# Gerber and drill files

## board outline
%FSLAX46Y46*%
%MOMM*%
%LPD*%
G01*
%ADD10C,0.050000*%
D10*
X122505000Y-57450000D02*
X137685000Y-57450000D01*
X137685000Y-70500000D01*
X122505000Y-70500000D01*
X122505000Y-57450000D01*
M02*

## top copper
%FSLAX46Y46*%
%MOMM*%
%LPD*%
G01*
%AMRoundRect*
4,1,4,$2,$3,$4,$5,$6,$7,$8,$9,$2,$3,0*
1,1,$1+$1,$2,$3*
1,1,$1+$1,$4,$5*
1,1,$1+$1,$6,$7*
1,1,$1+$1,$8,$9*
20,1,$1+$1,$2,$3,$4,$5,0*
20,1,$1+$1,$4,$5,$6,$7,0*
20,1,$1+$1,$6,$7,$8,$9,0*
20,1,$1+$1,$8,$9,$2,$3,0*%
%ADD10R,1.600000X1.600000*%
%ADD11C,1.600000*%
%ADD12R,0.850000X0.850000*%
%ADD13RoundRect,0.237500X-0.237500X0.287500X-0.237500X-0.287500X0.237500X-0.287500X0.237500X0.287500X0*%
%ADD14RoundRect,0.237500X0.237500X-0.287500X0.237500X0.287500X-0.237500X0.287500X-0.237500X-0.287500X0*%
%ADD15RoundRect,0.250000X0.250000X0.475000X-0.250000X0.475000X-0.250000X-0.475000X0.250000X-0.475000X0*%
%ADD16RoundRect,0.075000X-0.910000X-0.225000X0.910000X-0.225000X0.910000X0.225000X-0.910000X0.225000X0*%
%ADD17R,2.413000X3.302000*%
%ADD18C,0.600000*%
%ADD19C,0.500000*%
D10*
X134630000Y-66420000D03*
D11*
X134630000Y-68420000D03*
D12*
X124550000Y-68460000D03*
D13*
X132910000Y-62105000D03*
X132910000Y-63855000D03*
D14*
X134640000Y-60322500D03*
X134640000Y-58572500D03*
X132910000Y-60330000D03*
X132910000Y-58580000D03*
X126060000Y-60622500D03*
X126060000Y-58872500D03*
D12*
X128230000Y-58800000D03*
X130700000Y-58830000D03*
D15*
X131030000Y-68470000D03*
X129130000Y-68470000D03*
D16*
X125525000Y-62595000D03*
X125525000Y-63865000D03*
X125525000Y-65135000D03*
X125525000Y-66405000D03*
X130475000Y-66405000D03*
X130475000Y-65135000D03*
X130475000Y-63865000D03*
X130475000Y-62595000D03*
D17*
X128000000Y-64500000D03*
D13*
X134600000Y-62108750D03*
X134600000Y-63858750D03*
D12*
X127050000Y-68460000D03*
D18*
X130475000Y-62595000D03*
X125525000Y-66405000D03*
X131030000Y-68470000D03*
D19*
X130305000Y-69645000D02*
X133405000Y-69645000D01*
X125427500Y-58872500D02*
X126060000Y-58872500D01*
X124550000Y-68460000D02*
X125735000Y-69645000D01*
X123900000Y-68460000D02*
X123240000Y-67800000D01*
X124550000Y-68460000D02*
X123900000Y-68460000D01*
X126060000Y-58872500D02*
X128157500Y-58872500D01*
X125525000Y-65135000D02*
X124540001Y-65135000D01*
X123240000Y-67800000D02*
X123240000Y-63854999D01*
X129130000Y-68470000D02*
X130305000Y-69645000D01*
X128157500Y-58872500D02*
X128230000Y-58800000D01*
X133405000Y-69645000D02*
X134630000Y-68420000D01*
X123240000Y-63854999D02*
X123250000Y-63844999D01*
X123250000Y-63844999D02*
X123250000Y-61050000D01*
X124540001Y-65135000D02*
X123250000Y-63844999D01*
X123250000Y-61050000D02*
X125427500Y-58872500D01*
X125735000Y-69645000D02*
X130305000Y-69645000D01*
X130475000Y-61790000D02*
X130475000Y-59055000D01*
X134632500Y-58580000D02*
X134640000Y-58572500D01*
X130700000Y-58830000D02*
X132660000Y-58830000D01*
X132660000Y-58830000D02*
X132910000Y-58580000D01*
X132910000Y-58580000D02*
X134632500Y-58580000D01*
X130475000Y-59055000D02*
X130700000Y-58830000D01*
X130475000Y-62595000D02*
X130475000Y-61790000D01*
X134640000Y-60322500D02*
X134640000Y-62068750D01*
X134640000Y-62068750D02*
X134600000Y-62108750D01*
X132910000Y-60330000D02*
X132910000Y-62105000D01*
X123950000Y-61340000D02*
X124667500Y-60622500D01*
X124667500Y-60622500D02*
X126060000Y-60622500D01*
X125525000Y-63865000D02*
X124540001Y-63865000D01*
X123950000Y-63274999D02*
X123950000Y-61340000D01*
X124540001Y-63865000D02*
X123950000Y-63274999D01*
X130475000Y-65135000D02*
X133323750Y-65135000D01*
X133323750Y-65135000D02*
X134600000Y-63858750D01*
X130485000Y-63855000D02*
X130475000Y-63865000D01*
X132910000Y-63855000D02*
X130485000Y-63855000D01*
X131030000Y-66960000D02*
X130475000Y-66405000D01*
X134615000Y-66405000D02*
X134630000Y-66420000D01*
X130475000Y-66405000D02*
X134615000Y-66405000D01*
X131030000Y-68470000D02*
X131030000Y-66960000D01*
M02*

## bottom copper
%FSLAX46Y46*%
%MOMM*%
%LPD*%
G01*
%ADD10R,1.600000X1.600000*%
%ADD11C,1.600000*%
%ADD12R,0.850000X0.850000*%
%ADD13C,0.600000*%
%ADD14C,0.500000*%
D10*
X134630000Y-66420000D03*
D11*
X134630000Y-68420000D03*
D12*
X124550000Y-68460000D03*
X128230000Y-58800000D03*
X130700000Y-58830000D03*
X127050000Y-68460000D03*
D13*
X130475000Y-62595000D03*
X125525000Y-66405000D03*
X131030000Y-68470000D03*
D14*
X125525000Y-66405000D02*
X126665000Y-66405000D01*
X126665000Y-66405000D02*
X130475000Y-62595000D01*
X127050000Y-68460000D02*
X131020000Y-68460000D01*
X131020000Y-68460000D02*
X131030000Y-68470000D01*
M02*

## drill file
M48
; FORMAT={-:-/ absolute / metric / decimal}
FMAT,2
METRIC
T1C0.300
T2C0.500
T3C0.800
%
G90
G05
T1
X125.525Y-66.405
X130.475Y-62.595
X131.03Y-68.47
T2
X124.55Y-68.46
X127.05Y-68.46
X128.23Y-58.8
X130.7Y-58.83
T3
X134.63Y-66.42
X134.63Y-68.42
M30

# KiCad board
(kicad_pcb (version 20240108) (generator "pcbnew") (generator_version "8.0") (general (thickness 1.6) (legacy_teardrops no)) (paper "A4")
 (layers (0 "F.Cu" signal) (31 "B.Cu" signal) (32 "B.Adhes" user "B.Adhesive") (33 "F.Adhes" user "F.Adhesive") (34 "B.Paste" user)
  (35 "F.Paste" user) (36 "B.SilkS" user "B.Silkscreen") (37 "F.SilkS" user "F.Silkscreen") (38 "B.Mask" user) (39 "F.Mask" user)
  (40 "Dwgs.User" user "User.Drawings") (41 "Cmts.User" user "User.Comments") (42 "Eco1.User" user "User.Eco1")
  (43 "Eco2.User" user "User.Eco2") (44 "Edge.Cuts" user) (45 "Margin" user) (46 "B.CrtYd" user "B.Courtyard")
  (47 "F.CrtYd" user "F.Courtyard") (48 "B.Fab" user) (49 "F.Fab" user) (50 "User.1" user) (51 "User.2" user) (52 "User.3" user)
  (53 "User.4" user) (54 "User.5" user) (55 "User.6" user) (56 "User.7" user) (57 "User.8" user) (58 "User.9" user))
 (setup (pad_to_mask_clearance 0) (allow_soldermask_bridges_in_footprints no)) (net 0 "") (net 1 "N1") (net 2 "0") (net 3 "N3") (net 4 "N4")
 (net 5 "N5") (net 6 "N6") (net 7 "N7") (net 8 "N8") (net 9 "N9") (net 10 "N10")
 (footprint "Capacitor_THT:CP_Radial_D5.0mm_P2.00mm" (layer "F.Cu") (at 134.63 66.42 -90)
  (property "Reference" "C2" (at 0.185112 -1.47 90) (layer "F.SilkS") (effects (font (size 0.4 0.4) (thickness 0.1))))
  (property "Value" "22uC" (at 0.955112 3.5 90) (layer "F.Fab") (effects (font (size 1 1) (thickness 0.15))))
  (pad "1" thru_hole rect (at 0 0 270) (size 1.6 1.6) (drill 0.8) (layers "*.Cu" "*.Mask") (remove_unused_layers no) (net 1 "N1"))
  (pad "2" thru_hole circle (at 2 0 270) (size 1.6 1.6) (drill 0.8) (layers "*.Cu" "*.Mask") (remove_unused_layers no) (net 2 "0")))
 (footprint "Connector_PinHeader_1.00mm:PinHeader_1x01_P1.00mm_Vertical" (layer "F.Cu") (at 124.55 68.46)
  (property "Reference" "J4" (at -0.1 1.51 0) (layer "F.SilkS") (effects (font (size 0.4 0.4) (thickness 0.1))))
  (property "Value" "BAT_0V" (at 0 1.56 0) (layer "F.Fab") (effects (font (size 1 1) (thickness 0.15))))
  (pad "1" thru_hole rect (at 0 0) (size 0.85 0.85) (drill 0.5) (layers "*.Cu" "*.Mask") (remove_unused_layers no) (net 2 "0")))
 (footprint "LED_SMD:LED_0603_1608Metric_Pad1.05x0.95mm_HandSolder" (layer "F.Cu") (at 132.91 62.98 -90)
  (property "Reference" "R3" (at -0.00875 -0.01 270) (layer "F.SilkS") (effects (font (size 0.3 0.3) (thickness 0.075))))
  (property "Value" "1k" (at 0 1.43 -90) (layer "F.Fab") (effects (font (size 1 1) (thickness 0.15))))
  (pad "1" smd roundrect (at -0.875 0 270) (size 1.05 0.95) (layers "F.Cu" "F.Paste" "F.Mask") (roundrect_rratio 0.25) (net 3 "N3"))
  (pad "2" smd roundrect (at 0.875 0 270) (size 1.05 0.95) (layers "F.Cu" "F.Paste" "F.Mask") (roundrect_rratio 0.25) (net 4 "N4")))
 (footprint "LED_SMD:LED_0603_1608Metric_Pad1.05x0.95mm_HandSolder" (layer "F.Cu") (at 134.64 59.4475 90)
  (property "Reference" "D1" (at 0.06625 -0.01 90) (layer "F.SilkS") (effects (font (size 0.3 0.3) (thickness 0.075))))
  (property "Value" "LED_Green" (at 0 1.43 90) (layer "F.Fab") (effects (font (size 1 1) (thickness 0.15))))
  (pad "1" smd roundrect (at -0.875 0 90) (size 1.05 0.95) (layers "F.Cu" "F.Paste" "F.Mask") (roundrect_rratio 0.25) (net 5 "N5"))
  (pad "2" smd roundrect (at 0.875 0 90) (size 1.05 0.95) (layers "F.Cu" "F.Paste" "F.Mask") (roundrect_rratio 0.25) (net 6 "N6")))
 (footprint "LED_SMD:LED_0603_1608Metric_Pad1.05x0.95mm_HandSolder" (layer "F.Cu") (at 132.91 59.455 90)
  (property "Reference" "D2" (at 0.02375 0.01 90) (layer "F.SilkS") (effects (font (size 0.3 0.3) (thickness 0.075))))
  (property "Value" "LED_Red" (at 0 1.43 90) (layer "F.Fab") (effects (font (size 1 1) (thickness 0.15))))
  (pad "1" smd roundrect (at -0.875 0 90) (size 1.05 0.95) (layers "F.Cu" "F.Paste" "F.Mask") (roundrect_rratio 0.25) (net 3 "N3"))
  (pad "2" smd roundrect (at 0.875 0 90) (size 1.05 0.95) (layers "F.Cu" "F.Paste" "F.Mask") (roundrect_rratio 0.25) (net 6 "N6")))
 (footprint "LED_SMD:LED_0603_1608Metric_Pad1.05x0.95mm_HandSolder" (layer "F.Cu") (at 126.06 59.7475 90)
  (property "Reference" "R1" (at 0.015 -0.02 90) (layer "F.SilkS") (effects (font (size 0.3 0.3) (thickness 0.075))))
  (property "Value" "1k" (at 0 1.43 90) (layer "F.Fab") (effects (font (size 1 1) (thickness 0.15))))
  (pad "1" smd roundrect (at -0.875 0 90) (size 1.05 0.95) (layers "F.Cu" "F.Paste" "F.Mask") (roundrect_rratio 0.25) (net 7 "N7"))
  (pad "2" smd roundrect (at 0.875 0 90) (size 1.05 0.95) (layers "F.Cu" "F.Paste" "F.Mask") (roundrect_rratio 0.25) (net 2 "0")))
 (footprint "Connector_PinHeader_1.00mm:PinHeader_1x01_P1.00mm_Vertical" (layer "F.Cu") (at 128.23 58.8)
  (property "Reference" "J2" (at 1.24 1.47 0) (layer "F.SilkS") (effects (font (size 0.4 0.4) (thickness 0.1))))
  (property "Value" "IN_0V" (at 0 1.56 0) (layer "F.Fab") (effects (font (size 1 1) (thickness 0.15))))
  (pad "1" thru_hole rect (at 0 0) (size 0.85 0.85) (drill 0.5) (layers "*.Cu" "*.Mask") (remove_unused_layers no) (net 2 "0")))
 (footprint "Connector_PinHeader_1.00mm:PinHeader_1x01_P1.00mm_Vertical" (layer "F.Cu") (at 130.7 58.83)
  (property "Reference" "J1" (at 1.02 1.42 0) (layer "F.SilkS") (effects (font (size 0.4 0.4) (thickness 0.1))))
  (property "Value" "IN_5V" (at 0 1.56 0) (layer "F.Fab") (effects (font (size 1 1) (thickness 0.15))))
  (pad "1" thru_hole rect (at 0 0) (size 0.85 0.85) (drill 0.5) (layers "*.Cu" "*.Mask") (remove_unused_layers no) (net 6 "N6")))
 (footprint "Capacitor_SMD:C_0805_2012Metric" (layer "F.Cu") (at 130.08 68.47 180)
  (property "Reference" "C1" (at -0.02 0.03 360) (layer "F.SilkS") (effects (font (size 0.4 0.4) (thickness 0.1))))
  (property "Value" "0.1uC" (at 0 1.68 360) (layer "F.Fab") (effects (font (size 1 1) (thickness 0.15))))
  (pad "1" smd roundrect (at -0.95 0 180) (size 1 1.45) (layers "F.Cu" "F.Paste" "F.Mask") (roundrect_rratio 0.25) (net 1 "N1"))
  (pad "2" smd roundrect (at 0.95 0 180) (size 1 1.45) (layers "F.Cu" "F.Paste" "F.Mask") (roundrect_rratio 0.25) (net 2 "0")))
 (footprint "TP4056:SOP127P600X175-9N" (layer "F.Cu") (at 128 64.5)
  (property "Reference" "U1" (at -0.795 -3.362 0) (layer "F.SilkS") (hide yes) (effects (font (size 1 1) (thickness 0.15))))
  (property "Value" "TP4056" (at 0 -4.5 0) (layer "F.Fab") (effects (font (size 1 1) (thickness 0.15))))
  (pad "1" smd roundrect (at -2.475 -1.905) (size 1.97 0.6) (layers "F.Cu" "F.Paste" "F.Mask") (roundrect_rratio 0.125) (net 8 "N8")
   (solder_mask_margin 0.102))
  (pad "2" smd roundrect (at -2.475 -0.635) (size 1.97 0.6) (layers "F.Cu" "F.Paste" "F.Mask") (roundrect_rratio 0.125) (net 7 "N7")
   (solder_mask_margin 0.102))
  (pad "3" smd roundrect (at -2.475 0.635) (size 1.97 0.6) (layers "F.Cu" "F.Paste" "F.Mask") (roundrect_rratio 0.125) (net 2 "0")
   (solder_mask_margin 0.102))
  (pad "4" smd roundrect (at -2.475 1.905) (size 1.97 0.6) (layers "F.Cu" "F.Paste" "F.Mask") (roundrect_rratio 0.125) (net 6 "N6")
   (solder_mask_margin 0.102))
  (pad "5" smd roundrect (at 2.475 1.905) (size 1.97 0.6) (layers "F.Cu" "F.Paste" "F.Mask") (roundrect_rratio 0.125) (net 1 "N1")
   (solder_mask_margin 0.102))
  (pad "6" smd roundrect (at 2.475 0.635) (size 1.97 0.6) (layers "F.Cu" "F.Paste" "F.Mask") (roundrect_rratio 0.125) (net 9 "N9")
   (solder_mask_margin 0.102))
  (pad "7" smd roundrect (at 2.475 -0.635) (size 1.97 0.6) (layers "F.Cu" "F.Paste" "F.Mask") (roundrect_rratio 0.125) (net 4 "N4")
   (solder_mask_margin 0.102))
  (pad "8" smd roundrect (at 2.475 -1.905) (size 1.97 0.6) (layers "F.Cu" "F.Paste" "F.Mask") (roundrect_rratio 0.125) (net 6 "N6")
   (solder_mask_margin 0.102))
  (pad "9" smd rect (at 0 0) (size 2.413 3.302) (layers "F.Cu" "F.Mask") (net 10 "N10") (solder_mask_margin 0.102)))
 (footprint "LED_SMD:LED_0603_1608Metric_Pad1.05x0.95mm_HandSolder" (layer "F.Cu") (at 134.6 62.98375 -90)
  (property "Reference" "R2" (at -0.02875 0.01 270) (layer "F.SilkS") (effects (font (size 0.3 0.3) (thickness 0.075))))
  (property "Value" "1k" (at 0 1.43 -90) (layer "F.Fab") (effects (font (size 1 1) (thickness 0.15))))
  (pad "1" smd roundrect (at -0.875 0 270) (size 1.05 0.95) (layers "F.Cu" "F.Paste" "F.Mask") (roundrect_rratio 0.25) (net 5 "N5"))
  (pad "2" smd roundrect (at 0.875 0 270) (size 1.05 0.95) (layers "F.Cu" "F.Paste" "F.Mask") (roundrect_rratio 0.25) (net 9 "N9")))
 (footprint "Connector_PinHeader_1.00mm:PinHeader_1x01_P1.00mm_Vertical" (layer "F.Cu") (at 127.05 68.46)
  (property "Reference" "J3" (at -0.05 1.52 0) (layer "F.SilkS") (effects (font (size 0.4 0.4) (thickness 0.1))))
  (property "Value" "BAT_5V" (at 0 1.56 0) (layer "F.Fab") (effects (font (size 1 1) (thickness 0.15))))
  (pad "1" thru_hole rect (at 0 0) (size 0.85 0.85) (drill 0.5) (layers "*.Cu" "*.Mask") (remove_unused_layers no) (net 1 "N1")))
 (gr_rect (start 122.505 57.45) (end 137.685 70.5) (stroke (width 0.05) (type default)) (fill none) (layer "Edge.Cuts"))
 (segment (start 130.305 69.645) (end 133.405 69.645) (width 0.5) (layer "F.Cu") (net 2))
 (segment (start 125.4275 58.8725) (end 126.06 58.8725) (width 0.5) (layer "F.Cu") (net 2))
 (segment (start 124.55 68.46) (end 125.735 69.645) (width 0.5) (layer "F.Cu") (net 2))
 (segment (start 123.9 68.46) (end 123.24 67.8) (width 0.5) (layer "F.Cu") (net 2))
 (segment (start 124.55 68.46) (end 123.9 68.46) (width 0.5) (layer "F.Cu") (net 2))
 (segment (start 126.06 58.8725) (end 128.1575 58.8725) (width 0.5) (layer "F.Cu") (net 2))
 (segment (start 125.525 65.135) (end 124.540001 65.135) (width 0.5) (layer "F.Cu") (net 2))
 (segment (start 123.24 67.8) (end 123.24 63.854999) (width 0.5) (layer "F.Cu") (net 2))
 (segment (start 129.13 68.47) (end 130.305 69.645) (width 0.5) (layer "F.Cu") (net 2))
 (segment (start 128.1575 58.8725) (end 128.23 58.8) (width 0.5) (layer "F.Cu") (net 2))
 (segment (start 133.405 69.645) (end 134.63 68.42) (width 0.5) (layer "F.Cu") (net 2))
 (segment (start 123.24 63.854999) (end 123.25 63.844999) (width 0.5) (layer "F.Cu") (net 2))
 (segment (start 123.25 63.844999) (end 123.25 61.05) (width 0.5) (layer "F.Cu") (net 2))
 (segment (start 124.540001 65.135) (end 123.25 63.844999) (width 0.5) (layer "F.Cu") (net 2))
 (segment (start 123.25 61.05) (end 125.4275 58.8725) (width 0.5) (layer "F.Cu") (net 2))
 (segment (start 125.735 69.645) (end 130.305 69.645) (width 0.5) (layer "F.Cu") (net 2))
 (segment (start 130.475 61.79) (end 130.475 59.055) (width 0.5) (layer "F.Cu") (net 6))
 (segment (start 134.6325 58.58) (end 134.64 58.5725) (width 0.5) (layer "F.Cu") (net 6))
 (segment (start 130.7 58.83) (end 132.66 58.83) (width 0.5) (layer "F.Cu") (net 6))
 (segment (start 132.66 58.83) (end 132.91 58.58) (width 0.5) (layer "F.Cu") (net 6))
 (segment (start 132.91 58.58) (end 134.6325 58.58) (width 0.5) (layer "F.Cu") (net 6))
 (segment (start 130.475 59.055) (end 130.7 58.83) (width 0.5) (layer "F.Cu") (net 6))
 (segment (start 130.475 62.595) (end 130.475 61.79) (width 0.5) (layer "F.Cu") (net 6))
 (via (at 130.475 62.595) (size 0.6) (drill 0.3) (layers "F.Cu" "B.Cu") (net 6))
 (via (at 125.525 66.405) (size 0.6) (drill 0.3) (layers "F.Cu" "B.Cu") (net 6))
 (segment (start 125.525 66.405) (end 126.665 66.405) (width 0.5) (layer "B.Cu") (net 6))
 (segment (start 126.665 66.405) (end 130.475 62.595) (width 0.5) (layer "B.Cu") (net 6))
 (segment (start 134.64 60.3225) (end 134.64 62.06875) (width 0.5) (layer "F.Cu") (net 5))
 (segment (start 134.64 62.06875) (end 134.6 62.10875) (width 0.5) (layer "F.Cu") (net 5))
 (segment (start 132.91 60.33) (end 132.91 62.105) (width 0.5) (layer "F.Cu") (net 3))
 (segment (start 123.95 61.34) (end 124.6675 60.6225) (width 0.5) (layer "F.Cu") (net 7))
 (segment (start 124.6675 60.6225) (end 126.06 60.6225) (width 0.5) (layer "F.Cu") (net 7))
 (segment (start 125.525 63.865) (end 124.540001 63.865) (width 0.5) (layer "F.Cu") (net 7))
 (segment (start 123.95 63.274999) (end 123.95 61.34) (width 0.5) (layer "F.Cu") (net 7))
 (segment (start 124.540001 63.865) (end 123.95 63.274999) (width 0.5) (layer "F.Cu") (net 7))
 (segment (start 130.475 65.135) (end 133.32375 65.135) (width 0.5) (layer "F.Cu") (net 9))
 (segment (start 133.32375 65.135) (end 134.6 63.85875) (width 0.5) (layer "F.Cu") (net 9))
 (segment (start 130.485 63.855) (end 130.475 63.865) (width 0.5) (layer "F.Cu") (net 4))
 (segment (start 132.91 63.855) (end 130.485 63.855) (width 0.5) (layer "F.Cu") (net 4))
 (segment (start 131.03 66.96) (end 130.475 66.405) (width 0.5) (layer "F.Cu") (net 1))
 (segment (start 134.615 66.405) (end 134.63 66.42) (width 0.5) (layer "F.Cu") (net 1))
 (segment (start 130.475 66.405) (end 134.615 66.405) (width 0.5) (layer "F.Cu") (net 1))
 (segment (start 131.03 68.47) (end 131.03 66.96) (width 0.5) (layer "F.Cu") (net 1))
 (via (at 131.03 68.47) (size 0.6) (drill 0.3) (layers "F.Cu" "B.Cu") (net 1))
 (segment (start 127.05 68.46) (end 131.02 68.46) (width 0.5) (layer "B.Cu") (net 1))
 (segment (start 131.02 68.46) (end 131.03 68.47) (width 0.5) (layer "B.Cu") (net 1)))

